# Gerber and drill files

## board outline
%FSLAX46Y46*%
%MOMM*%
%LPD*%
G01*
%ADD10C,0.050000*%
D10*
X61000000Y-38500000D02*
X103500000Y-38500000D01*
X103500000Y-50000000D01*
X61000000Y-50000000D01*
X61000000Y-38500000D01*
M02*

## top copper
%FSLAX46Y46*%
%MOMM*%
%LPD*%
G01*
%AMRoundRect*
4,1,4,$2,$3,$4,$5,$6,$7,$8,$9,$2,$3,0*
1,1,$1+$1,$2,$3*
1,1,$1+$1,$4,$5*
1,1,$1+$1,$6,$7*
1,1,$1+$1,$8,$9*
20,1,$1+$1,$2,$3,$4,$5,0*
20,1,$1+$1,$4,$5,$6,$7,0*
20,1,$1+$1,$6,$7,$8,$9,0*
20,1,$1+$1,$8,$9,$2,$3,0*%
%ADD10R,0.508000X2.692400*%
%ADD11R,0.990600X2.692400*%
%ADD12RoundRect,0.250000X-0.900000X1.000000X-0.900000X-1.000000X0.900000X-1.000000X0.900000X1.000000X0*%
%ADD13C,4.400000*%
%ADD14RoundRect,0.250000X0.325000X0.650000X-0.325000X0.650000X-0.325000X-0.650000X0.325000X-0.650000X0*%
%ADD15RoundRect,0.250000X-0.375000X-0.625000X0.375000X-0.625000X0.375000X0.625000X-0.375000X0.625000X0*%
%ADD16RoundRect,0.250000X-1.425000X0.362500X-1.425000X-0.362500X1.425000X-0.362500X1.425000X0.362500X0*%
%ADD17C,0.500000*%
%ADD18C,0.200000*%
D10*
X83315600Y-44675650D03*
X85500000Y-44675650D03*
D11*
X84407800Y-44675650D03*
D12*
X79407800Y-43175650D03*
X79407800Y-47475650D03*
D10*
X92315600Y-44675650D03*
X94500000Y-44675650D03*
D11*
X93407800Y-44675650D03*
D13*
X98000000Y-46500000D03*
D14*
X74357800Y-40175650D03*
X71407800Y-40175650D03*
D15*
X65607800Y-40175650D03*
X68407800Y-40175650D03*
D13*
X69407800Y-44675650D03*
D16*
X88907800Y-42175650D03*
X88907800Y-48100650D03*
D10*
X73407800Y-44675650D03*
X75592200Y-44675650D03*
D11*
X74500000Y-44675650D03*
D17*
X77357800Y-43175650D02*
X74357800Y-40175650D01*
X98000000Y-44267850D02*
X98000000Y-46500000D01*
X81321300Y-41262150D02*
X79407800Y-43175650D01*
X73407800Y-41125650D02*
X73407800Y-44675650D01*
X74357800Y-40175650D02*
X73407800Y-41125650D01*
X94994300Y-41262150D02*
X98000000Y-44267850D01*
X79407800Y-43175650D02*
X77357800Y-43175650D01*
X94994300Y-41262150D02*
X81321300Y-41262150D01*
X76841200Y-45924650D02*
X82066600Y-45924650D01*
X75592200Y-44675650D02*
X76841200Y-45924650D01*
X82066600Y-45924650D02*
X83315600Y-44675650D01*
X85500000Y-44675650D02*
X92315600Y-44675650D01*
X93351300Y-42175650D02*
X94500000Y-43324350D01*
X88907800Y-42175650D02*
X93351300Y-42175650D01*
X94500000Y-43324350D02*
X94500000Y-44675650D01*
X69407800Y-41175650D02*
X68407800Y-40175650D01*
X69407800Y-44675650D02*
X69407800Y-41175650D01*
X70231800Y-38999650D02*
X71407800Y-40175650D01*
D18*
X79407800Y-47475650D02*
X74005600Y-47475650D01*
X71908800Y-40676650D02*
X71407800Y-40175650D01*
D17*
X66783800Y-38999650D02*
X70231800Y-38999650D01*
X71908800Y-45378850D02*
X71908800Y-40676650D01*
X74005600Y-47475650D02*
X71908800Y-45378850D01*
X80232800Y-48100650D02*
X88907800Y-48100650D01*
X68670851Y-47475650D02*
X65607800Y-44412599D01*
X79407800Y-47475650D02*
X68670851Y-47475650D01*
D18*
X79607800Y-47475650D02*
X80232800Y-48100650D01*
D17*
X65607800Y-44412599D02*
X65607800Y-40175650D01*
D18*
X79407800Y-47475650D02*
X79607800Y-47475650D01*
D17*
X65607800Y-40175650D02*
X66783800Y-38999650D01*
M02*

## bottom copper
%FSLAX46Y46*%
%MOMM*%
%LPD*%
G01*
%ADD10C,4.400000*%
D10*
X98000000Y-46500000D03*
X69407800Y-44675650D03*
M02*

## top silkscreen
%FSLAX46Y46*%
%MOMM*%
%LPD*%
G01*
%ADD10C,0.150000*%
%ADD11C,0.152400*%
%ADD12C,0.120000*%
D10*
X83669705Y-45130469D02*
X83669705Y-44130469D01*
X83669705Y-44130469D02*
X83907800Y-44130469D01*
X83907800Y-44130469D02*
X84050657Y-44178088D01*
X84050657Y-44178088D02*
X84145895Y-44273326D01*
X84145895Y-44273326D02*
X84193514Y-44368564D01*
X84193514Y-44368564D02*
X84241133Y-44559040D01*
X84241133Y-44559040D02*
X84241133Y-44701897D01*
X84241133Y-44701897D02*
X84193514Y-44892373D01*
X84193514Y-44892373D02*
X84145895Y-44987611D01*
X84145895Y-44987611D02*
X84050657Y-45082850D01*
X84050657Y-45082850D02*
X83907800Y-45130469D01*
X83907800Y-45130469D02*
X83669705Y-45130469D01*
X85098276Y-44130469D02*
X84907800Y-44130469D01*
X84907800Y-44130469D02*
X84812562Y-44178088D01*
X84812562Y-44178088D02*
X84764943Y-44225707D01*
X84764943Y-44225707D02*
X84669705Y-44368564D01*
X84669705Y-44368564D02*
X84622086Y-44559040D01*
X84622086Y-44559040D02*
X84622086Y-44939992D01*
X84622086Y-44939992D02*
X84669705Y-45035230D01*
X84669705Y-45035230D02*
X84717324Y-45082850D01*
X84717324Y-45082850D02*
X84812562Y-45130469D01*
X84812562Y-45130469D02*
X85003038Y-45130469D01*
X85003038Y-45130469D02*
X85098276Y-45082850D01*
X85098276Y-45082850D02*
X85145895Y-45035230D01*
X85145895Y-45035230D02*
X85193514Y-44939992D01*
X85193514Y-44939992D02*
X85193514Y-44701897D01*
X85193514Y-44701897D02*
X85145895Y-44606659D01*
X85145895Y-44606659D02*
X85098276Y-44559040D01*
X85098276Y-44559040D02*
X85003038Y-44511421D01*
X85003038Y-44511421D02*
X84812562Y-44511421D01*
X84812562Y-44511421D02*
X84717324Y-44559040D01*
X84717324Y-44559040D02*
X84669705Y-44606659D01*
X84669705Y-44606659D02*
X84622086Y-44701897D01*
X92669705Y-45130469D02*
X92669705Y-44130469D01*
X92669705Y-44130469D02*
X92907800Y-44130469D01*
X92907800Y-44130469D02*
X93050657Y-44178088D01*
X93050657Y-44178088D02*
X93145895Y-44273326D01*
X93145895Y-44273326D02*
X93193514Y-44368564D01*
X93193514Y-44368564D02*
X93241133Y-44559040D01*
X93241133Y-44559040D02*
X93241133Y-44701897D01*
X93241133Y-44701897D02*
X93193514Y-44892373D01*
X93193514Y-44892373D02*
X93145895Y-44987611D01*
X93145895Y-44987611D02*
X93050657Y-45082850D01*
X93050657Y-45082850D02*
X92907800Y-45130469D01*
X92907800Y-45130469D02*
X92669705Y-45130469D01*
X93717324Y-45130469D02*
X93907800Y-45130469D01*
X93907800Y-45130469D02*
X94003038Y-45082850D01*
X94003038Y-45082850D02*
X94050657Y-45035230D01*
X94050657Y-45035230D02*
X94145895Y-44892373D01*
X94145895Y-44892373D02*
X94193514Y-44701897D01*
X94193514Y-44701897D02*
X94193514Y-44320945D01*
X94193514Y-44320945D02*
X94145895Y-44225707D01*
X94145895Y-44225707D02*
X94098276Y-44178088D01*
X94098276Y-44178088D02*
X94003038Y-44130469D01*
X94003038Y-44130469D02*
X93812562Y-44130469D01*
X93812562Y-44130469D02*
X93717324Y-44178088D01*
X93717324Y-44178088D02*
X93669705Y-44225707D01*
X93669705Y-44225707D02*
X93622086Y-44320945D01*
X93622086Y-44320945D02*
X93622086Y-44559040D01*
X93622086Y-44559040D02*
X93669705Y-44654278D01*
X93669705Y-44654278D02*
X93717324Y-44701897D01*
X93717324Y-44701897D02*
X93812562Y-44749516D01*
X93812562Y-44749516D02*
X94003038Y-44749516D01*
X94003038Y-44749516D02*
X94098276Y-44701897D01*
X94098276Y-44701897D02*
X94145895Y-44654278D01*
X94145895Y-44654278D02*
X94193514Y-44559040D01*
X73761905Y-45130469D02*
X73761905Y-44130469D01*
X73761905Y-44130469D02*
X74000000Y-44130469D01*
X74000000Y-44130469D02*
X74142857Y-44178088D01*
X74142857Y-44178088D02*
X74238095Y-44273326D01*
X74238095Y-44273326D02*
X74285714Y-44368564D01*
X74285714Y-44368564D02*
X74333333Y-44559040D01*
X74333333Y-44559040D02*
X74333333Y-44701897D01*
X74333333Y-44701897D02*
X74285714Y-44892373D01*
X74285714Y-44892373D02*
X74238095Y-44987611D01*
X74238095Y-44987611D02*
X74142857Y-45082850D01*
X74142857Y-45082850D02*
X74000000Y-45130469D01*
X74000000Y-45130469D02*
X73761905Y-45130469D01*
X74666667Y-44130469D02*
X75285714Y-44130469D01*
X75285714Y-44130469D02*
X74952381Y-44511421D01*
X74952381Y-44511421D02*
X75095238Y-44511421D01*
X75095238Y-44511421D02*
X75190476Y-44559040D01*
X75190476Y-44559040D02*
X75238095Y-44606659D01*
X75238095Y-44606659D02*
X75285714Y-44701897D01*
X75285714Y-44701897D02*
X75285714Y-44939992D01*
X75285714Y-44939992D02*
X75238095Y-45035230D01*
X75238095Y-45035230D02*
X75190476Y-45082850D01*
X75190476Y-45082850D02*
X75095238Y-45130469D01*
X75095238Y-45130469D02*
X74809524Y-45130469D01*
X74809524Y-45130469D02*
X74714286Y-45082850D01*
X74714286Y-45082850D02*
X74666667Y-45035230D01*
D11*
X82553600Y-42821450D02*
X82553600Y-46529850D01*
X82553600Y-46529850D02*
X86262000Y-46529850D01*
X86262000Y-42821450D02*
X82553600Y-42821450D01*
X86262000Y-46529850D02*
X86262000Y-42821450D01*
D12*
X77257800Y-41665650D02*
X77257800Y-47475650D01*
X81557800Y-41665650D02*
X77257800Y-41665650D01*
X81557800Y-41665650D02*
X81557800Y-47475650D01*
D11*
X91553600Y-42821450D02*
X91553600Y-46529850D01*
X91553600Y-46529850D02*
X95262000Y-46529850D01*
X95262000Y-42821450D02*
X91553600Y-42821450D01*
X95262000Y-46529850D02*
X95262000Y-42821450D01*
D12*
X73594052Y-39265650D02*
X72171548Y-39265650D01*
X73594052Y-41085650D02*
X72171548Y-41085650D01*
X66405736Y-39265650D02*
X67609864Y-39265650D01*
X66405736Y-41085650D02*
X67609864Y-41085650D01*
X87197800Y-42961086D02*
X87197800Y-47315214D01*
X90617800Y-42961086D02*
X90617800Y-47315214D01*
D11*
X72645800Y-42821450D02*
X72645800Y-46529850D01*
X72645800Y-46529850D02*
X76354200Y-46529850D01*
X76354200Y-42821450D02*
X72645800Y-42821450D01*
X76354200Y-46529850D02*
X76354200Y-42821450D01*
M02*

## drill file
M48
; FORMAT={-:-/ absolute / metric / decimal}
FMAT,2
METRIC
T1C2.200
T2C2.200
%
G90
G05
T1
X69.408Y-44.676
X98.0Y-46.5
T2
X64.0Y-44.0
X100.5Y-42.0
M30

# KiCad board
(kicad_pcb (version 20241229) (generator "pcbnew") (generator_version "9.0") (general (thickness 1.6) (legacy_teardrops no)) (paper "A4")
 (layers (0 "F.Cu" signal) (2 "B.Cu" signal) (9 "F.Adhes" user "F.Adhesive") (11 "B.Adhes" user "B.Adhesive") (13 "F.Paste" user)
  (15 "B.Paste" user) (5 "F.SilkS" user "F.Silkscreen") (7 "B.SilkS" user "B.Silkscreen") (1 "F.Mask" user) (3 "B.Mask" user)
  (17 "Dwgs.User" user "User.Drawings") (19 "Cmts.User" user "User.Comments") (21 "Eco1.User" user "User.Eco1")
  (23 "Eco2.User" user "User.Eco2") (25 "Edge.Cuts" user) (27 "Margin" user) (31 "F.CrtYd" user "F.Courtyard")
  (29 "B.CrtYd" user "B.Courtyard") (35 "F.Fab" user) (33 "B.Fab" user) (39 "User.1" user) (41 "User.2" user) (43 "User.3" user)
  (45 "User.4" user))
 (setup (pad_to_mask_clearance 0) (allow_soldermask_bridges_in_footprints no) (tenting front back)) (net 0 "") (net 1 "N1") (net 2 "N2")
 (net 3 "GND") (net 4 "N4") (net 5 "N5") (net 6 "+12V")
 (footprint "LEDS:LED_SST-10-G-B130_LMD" (layer "F.Cu") (at 84.4078 44.67565)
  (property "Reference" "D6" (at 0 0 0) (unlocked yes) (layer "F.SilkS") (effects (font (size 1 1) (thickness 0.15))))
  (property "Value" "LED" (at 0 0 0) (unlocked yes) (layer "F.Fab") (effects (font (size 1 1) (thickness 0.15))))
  (fp_line (start -1.8542 -1.8542) (end -1.8542 1.8542) (stroke (width 0.1524) (type solid)) (layer "F.SilkS"))
  (fp_line (start -1.8542 1.8542) (end 1.8542 1.8542) (stroke (width 0.1524) (type solid)) (layer "F.SilkS"))
  (fp_line (start 1.8542 -1.8542) (end -1.8542 -1.8542) (stroke (width 0.1524) (type solid)) (layer "F.SilkS"))
  (fp_line (start 1.8542 1.8542) (end 1.8542 -1.8542) (stroke (width 0.1524) (type solid)) (layer "F.SilkS"))
  (pad "1" smd rect (at -1.0922 0) (size 0.508 2.6924) (layers "F.Cu" "F.Mask" "F.Paste") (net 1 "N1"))
  (pad "2" smd rect (at 1.0922 0) (size 0.508 2.6924) (layers "F.Cu" "F.Mask" "F.Paste") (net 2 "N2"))
  (pad "3" smd rect (at 0 0) (size 0.9906 2.6924) (layers "F.Cu" "F.Mask" "F.Paste")))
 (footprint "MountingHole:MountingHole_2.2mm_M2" (layer "F.Cu") (at 64 44)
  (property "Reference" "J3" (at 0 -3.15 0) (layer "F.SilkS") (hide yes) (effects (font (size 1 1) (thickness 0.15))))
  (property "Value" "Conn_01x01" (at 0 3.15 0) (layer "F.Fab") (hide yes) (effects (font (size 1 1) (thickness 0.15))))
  (pad "" np_thru_hole circle (at 0 0) (size 2.2 2.2) (drill 2.2) (layers "*.Cu" "*.Mask")))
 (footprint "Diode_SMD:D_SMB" (layer "F.Cu") (at 79.4078 45.32565 -90)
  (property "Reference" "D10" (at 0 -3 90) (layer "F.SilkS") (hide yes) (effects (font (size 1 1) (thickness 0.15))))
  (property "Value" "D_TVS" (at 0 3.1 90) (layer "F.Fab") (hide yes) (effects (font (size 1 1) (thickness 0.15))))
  (fp_line (start -3.66 2.15) (end 2.15 2.15) (stroke (width 0.12) (type solid)) (layer "F.SilkS"))
  (fp_line (start -3.66 -2.15) (end -3.66 2.15) (stroke (width 0.12) (type solid)) (layer "F.SilkS"))
  (fp_line (start -3.66 -2.15) (end 2.15 -2.15) (stroke (width 0.12) (type solid)) (layer "F.SilkS"))
  (pad "1" smd roundrect (at -2.15 0 270) (size 2.5 2.3) (layers "F.Cu" "F.Mask" "F.Paste") (roundrect_rratio 0.1086956522) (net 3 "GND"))
  (pad "2" smd roundrect (at 2.15 0 270) (size 2.5 2.3) (layers "F.Cu" "F.Mask" "F.Paste") (roundrect_rratio 0.1086956522) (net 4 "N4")))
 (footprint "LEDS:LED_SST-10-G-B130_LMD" (layer "F.Cu") (at 93.4078 44.67565)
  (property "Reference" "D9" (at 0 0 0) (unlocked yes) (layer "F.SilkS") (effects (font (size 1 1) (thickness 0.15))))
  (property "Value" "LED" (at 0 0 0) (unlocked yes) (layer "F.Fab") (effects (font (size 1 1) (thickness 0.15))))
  (fp_line (start -1.8542 -1.8542) (end -1.8542 1.8542) (stroke (width 0.1524) (type solid)) (layer "F.SilkS"))
  (fp_line (start -1.8542 1.8542) (end 1.8542 1.8542) (stroke (width 0.1524) (type solid)) (layer "F.SilkS"))
  (fp_line (start 1.8542 -1.8542) (end -1.8542 -1.8542) (stroke (width 0.1524) (type solid)) (layer "F.SilkS"))
  (fp_line (start 1.8542 1.8542) (end 1.8542 -1.8542) (stroke (width 0.1524) (type solid)) (layer "F.SilkS"))
  (pad "1" smd rect (at -1.0922 0) (size 0.508 2.6924) (layers "F.Cu" "F.Mask" "F.Paste") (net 2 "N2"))
  (pad "2" smd rect (at 1.0922 0) (size 0.508 2.6924) (layers "F.Cu" "F.Mask" "F.Paste") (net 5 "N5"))
  (pad "3" smd rect (at 0 0) (size 0.9906 2.6924) (layers "F.Cu" "F.Mask" "F.Paste")))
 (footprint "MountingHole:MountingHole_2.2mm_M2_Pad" (layer "F.Cu") (at 98 46.5)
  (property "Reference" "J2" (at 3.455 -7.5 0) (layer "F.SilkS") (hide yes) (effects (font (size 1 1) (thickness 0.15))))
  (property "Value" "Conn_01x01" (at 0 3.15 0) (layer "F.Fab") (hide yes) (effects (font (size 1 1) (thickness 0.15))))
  (pad "1" thru_hole circle (at 0 0) (size 4.4 4.4) (drill 2.2) (layers "*.Cu" "*.Mask") (remove_unused_layers no) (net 3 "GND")
   (zone_connect 2)))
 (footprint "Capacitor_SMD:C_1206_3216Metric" (layer "F.Cu") (at 72.8828 40.17565 180)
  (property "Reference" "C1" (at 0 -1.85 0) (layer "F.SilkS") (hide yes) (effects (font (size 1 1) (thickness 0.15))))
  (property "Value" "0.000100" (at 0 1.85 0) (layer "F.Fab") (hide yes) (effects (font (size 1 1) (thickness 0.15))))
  (fp_line (start -0.711252 0.91) (end 0.711252 0.91) (stroke (width 0.12) (type solid)) (layer "F.SilkS"))
  (fp_line (start -0.711252 -0.91) (end 0.711252 -0.91) (stroke (width 0.12) (type solid)) (layer "F.SilkS"))
  (pad "1" smd roundrect (at -1.475 0 180) (size 1.15 1.8) (layers "F.Cu" "F.Mask" "F.Paste") (roundrect_rratio 0.217391) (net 3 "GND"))
  (pad "2" smd roundrect (at 1.475 0 180) (size 1.15 1.8) (layers "F.Cu" "F.Mask" "F.Paste") (roundrect_rratio 0.217391) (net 4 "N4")))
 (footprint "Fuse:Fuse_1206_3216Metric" (layer "F.Cu") (at 67.0078 40.17565)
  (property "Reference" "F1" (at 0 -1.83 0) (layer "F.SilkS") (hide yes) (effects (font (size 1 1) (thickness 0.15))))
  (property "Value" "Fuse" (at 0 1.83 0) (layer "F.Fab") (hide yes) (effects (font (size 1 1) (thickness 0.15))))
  (fp_line (start -0.602064 -0.91) (end 0.602064 -0.91) (stroke (width 0.12) (type solid)) (layer "F.SilkS"))
  (fp_line (start -0.602064 0.91) (end 0.602064 0.91) (stroke (width 0.12) (type solid)) (layer "F.SilkS"))
  (pad "1" smd roundrect (at -1.4 0) (size 1.25 1.75) (layers "F.Cu" "F.Mask" "F.Paste") (roundrect_rratio 0.2) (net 4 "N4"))
  (pad "2" smd roundrect (at 1.4 0) (size 1.25 1.75) (layers "F.Cu" "F.Mask" "F.Paste") (roundrect_rratio 0.2) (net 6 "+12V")))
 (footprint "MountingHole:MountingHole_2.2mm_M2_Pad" (layer "F.Cu") (at 69.4078 44.67565)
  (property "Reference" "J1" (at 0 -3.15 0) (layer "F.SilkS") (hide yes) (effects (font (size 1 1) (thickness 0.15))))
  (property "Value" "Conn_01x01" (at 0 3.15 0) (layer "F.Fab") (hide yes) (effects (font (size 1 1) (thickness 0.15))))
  (pad "1" thru_hole circle (at 0 0) (size 4.4 4.4) (drill 2.2) (layers "*.Cu" "*.Mask") (remove_unused_layers no) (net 6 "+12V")
   (zone_connect 2)))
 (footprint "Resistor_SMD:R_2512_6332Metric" (layer "F.Cu") (at 88.9078 45.13815 -90)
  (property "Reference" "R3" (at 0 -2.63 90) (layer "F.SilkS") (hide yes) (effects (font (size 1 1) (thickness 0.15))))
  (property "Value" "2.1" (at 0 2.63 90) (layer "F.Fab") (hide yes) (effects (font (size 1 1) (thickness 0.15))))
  (fp_line (start -2.177064 1.71) (end 2.177064 1.71) (stroke (width 0.12) (type solid)) (layer "F.SilkS"))
  (fp_line (start -2.177064 -1.71) (end 2.177064 -1.71) (stroke (width 0.12) (type solid)) (layer "F.SilkS"))
  (pad "1" smd roundrect (at -2.9625 0 270) (size 1.225 3.35) (layers "F.Cu" "F.Mask" "F.Paste") (roundrect_rratio 0.204082) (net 5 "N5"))
  (pad "2" smd roundrect (at 2.9625 0 270) (size 1.225 3.35) (layers "F.Cu" "F.Mask" "F.Paste") (roundrect_rratio 0.204082) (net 4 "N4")))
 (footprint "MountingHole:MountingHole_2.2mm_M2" (layer "F.Cu") (at 100.5 42)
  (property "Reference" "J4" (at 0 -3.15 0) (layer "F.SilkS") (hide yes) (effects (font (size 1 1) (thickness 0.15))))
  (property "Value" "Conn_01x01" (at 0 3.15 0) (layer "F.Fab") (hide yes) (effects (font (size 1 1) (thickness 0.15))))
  (pad "" np_thru_hole circle (at 0 0) (size 2.2 2.2) (drill 2.2) (layers "*.Cu" "*.Mask")))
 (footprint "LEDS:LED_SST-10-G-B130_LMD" (layer "F.Cu") (at 74.5 44.67565)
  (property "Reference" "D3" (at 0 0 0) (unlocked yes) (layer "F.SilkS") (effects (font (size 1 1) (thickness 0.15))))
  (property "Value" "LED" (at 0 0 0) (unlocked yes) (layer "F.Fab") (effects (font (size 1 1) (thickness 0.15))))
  (fp_line (start -1.8542 -1.8542) (end -1.8542 1.8542) (stroke (width 0.1524) (type solid)) (layer "F.SilkS"))
  (fp_line (start -1.8542 1.8542) (end 1.8542 1.8542) (stroke (width 0.1524) (type solid)) (layer "F.SilkS"))
  (fp_line (start 1.8542 -1.8542) (end -1.8542 -1.8542) (stroke (width 0.1524) (type solid)) (layer "F.SilkS"))
  (fp_line (start 1.8542 1.8542) (end 1.8542 -1.8542) (stroke (width 0.1524) (type solid)) (layer "F.SilkS"))
  (pad "1" smd rect (at -1.0922 0) (size 0.508 2.6924) (layers "F.Cu" "F.Mask" "F.Paste") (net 3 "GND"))
  (pad "2" smd rect (at 1.0922 0) (size 0.508 2.6924) (layers "F.Cu" "F.Mask" "F.Paste") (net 1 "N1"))
  (pad "3" smd rect (at 0 0) (size 0.9906 2.6924) (layers "F.Cu" "F.Mask" "F.Paste")))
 (gr_rect (start 61 38.5) (end 103.5 50) (stroke (width 0.05) (type default)) (fill no) (layer "Edge.Cuts"))
 (segment (start 77.3578 43.17565) (end 74.3578 40.17565) (width 0.5) (layer "F.Cu") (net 3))
 (segment (start 98 44.26785) (end 98 46.5) (width 0.5) (layer "F.Cu") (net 3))
 (segment (start 81.3213 41.26215) (end 79.4078 43.17565) (width 0.5) (layer "F.Cu") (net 3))
 (segment (start 73.4078 41.12565) (end 73.4078 44.67565) (width 0.5) (layer "F.Cu") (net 3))
 (segment (start 74.3578 40.17565) (end 73.4078 41.12565) (width 0.5) (layer "F.Cu") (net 3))
 (segment (start 94.9943 41.26215) (end 98 44.26785) (width 0.5) (layer "F.Cu") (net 3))
 (segment (start 79.4078 43.17565) (end 77.3578 43.17565) (width 0.5) (layer "F.Cu") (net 3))
 (segment (start 94.9943 41.26215) (end 81.3213 41.26215) (width 0.5) (layer "F.Cu") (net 3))
 (segment (start 76.8412 45.92465) (end 82.0666 45.92465) (width 0.5) (layer "F.Cu") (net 1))
 (segment (start 75.5922 44.67565) (end 76.8412 45.92465) (width 0.5) (layer "F.Cu") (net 1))
 (segment (start 82.0666 45.92465) (end 83.3156 44.67565) (width 0.5) (layer "F.Cu") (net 1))
 (segment (start 85.5 44.67565) (end 92.3156 44.67565) (width 0.5) (layer "F.Cu") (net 2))
 (segment (start 93.3513 42.17565) (end 94.5 43.32435) (width 0.5) (layer "F.Cu") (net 5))
 (segment (start 88.9078 42.17565) (end 93.3513 42.17565) (width 0.5) (layer "F.Cu") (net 5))
 (segment (start 94.5 43.32435) (end 94.5 44.67565) (width 0.5) (layer "F.Cu") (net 5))
 (segment (start 69.4078 41.17565) (end 68.4078 40.17565) (width 0.5) (layer "F.Cu") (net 6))
 (segment (start 69.4078 44.67565) (end 69.4078 41.17565) (width 0.5) (layer "F.Cu") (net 6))
 (segment (start 70.2318 38.99965) (end 71.4078 40.17565) (width 0.5) (layer "F.Cu") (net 4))
 (segment (start 79.4078 47.47565) (end 74.0056 47.47565) (width 0.2) (layer "F.Cu") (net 4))
 (segment (start 71.9088 40.67665) (end 71.4078 40.17565) (width 0.2) (layer "F.Cu") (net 4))
 (segment (start 66.7838 38.99965) (end 70.2318 38.99965) (width 0.5) (layer "F.Cu") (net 4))
 (segment (start 71.9088 45.37885) (end 71.9088 40.67665) (width 0.5) (layer "F.Cu") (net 4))
 (segment (start 74.0056 47.47565) (end 71.9088 45.37885) (width 0.5) (layer "F.Cu") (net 4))
 (segment (start 80.2328 48.10065) (end 88.9078 48.10065) (width 0.5) (layer "F.Cu") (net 4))
 (segment (start 68.670851 47.47565) (end 65.6078 44.412599) (width 0.5) (layer "F.Cu") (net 4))
 (segment (start 79.4078 47.47565) (end 68.670851 47.47565) (width 0.5) (layer "F.Cu") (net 4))
 (segment (start 79.6078 47.47565) (end 80.2328 48.10065) (width 0.2) (layer "F.Cu") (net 4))
 (segment (start 65.6078 44.412599) (end 65.6078 40.17565) (width 0.5) (layer "F.Cu") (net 4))
 (segment (start 79.4078 47.47565) (end 79.6078 47.47565) (width 0.2) (layer "F.Cu") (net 4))
 (segment (start 65.6078 40.17565) (end 66.7838 38.99965) (width 0.5) (layer "F.Cu") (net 4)))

